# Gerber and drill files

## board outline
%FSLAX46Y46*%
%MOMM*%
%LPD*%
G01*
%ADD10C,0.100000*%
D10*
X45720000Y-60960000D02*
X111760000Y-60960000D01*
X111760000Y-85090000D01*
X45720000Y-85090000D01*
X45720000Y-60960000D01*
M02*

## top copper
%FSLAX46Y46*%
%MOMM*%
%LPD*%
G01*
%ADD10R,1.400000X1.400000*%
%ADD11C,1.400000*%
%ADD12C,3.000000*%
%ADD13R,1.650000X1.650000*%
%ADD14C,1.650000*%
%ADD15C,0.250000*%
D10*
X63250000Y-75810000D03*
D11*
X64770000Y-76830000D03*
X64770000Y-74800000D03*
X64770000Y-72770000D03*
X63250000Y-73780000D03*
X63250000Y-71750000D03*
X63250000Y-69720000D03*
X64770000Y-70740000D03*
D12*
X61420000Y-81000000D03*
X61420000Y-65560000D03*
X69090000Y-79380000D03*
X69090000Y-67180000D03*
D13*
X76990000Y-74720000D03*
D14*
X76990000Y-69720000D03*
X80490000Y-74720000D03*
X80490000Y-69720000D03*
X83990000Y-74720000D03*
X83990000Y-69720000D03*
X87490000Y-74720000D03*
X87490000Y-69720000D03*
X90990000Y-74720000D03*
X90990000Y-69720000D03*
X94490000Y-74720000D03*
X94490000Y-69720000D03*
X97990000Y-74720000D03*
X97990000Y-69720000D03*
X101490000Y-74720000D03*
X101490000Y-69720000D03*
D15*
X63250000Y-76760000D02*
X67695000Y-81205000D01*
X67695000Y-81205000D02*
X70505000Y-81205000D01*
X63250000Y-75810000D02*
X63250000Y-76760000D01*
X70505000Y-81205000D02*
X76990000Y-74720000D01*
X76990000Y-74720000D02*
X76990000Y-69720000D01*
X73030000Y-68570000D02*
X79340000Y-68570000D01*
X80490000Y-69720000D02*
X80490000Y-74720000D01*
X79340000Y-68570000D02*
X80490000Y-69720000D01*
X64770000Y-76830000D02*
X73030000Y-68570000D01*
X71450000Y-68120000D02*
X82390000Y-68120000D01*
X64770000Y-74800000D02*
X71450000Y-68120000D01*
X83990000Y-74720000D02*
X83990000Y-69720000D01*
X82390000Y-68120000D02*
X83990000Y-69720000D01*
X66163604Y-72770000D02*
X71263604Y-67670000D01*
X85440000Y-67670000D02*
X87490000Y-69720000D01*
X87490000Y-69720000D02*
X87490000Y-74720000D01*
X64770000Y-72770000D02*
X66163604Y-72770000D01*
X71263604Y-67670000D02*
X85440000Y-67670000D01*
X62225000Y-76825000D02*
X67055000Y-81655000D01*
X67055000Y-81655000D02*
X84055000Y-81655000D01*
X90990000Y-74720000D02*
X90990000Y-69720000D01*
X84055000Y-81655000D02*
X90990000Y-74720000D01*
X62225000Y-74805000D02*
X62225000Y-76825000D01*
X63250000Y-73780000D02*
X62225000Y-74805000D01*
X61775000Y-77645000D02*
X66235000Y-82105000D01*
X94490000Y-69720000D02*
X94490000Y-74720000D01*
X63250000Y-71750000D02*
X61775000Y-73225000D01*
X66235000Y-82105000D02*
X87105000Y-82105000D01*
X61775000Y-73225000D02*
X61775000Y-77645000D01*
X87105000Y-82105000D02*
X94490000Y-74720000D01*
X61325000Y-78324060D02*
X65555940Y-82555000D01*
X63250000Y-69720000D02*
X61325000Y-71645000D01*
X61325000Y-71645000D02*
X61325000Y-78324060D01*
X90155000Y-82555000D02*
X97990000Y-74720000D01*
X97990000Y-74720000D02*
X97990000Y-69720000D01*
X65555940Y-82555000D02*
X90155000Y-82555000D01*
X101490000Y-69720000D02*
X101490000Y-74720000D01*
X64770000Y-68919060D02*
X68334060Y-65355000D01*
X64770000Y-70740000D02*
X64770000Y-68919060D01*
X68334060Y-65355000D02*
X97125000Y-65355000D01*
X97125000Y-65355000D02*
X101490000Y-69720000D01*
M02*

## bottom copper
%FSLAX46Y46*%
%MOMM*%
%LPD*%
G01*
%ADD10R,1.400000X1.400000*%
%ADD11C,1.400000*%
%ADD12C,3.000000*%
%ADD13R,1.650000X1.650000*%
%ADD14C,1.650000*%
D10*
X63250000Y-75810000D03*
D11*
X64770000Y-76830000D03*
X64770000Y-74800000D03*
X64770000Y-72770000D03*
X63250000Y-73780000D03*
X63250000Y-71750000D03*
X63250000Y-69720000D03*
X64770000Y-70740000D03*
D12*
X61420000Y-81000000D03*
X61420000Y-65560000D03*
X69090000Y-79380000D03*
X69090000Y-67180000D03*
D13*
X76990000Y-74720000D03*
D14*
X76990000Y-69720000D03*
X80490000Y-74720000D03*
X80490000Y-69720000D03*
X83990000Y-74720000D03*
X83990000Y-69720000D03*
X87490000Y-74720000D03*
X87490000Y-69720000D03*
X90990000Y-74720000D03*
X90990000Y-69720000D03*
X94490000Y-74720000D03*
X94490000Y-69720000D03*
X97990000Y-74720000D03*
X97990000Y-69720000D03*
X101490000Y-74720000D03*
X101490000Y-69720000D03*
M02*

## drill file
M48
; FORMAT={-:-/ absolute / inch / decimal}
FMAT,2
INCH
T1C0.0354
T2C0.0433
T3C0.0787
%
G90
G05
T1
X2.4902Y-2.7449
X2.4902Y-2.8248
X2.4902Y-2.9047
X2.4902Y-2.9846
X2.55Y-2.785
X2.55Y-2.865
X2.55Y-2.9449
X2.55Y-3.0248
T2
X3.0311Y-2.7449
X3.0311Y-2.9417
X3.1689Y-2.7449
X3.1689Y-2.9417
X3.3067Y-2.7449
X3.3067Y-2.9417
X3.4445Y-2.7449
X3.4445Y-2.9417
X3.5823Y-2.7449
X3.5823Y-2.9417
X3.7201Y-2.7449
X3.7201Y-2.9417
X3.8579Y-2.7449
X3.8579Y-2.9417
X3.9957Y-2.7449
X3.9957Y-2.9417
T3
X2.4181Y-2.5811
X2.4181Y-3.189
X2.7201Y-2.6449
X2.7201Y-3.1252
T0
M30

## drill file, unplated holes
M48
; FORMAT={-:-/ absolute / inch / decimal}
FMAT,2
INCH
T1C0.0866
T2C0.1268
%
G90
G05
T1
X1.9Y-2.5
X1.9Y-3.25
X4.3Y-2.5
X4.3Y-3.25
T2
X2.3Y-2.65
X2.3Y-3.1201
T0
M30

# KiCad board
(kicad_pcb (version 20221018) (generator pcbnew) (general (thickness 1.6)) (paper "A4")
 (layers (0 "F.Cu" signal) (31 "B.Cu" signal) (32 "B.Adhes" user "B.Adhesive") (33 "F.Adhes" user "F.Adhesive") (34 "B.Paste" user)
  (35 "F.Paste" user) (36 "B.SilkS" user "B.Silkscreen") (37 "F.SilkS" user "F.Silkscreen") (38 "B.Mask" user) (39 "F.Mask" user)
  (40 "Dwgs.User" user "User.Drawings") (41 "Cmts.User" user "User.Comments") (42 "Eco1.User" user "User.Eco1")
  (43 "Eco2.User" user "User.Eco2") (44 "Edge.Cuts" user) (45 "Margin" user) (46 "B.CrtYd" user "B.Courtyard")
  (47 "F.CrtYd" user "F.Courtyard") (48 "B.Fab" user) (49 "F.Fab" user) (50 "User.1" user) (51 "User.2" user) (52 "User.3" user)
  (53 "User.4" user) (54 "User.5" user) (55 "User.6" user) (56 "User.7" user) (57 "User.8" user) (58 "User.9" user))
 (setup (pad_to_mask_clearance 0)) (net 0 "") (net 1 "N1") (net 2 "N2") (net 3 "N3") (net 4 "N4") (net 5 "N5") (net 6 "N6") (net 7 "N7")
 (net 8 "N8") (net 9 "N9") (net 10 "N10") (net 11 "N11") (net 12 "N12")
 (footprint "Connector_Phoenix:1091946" (layer "F.Cu") (at 63.25 75.81 -90)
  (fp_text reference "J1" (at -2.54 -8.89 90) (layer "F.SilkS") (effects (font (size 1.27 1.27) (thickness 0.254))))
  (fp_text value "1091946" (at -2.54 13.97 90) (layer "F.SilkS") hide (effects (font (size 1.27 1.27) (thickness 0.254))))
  (pad "" np_thru_hole circle (at -8.5 4.83 270) (size 3.22 3.22) (drill 3.22) (layers "*.Cu" "*.Mask"))
  (pad "" np_thru_hole circle (at 3.44 4.83 270) (size 3.22 3.22) (drill 3.22) (layers "*.Cu" "*.Mask"))
  (pad "1" thru_hole rect (at 0 0 270) (size 1.4 1.4) (drill 0.9) (layers "*.Cu" "*.Mask") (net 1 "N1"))
  (pad "2" thru_hole circle (at 1.02 -1.52 270) (size 1.4 1.4) (drill 0.9) (layers "*.Cu" "*.Mask") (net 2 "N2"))
  (pad "3" thru_hole circle (at -1.01 -1.52 270) (size 1.4 1.4) (drill 0.9) (layers "*.Cu" "*.Mask") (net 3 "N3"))
  (pad "4" thru_hole circle (at -3.04 -1.52 270) (size 1.4 1.4) (drill 0.9) (layers "*.Cu" "*.Mask") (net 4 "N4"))
  (pad "5" thru_hole circle (at -2.03 0 270) (size 1.4 1.4) (drill 0.9) (layers "*.Cu" "*.Mask") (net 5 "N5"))
  (pad "6" thru_hole circle (at -4.06 0 270) (size 1.4 1.4) (drill 0.9) (layers "*.Cu" "*.Mask") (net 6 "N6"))
  (pad "7" thru_hole circle (at -6.09 0 270) (size 1.4 1.4) (drill 0.9) (layers "*.Cu" "*.Mask") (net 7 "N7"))
  (pad "8" thru_hole circle (at -5.07 -1.52 270) (size 1.4 1.4) (drill 0.9) (layers "*.Cu" "*.Mask") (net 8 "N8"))
  (pad "MH1" thru_hole circle (at 5.19 1.83 270) (size 3 3) (drill 2) (layers "*.Cu" "*.Mask") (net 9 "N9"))
  (pad "MH2" thru_hole circle (at -10.25 1.83 270) (size 3 3) (drill 2) (layers "*.Cu" "*.Mask") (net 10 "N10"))
  (pad "MH3" thru_hole circle (at 3.57 -5.84 270) (size 3 3) (drill 2) (layers "*.Cu" "*.Mask") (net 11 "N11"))
  (pad "MH4" thru_hole circle (at -8.63 -5.84 270) (size 3 3) (drill 2) (layers "*.Cu" "*.Mask") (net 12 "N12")))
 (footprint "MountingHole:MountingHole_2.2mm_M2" (layer "F.Cu") (at 109.22 63.5)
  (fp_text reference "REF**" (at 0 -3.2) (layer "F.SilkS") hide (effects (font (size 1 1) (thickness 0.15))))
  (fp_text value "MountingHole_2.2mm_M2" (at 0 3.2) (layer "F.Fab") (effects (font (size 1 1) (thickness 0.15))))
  (pad "" np_thru_hole circle (at 0 0) (size 2.2 2.2) (drill 2.2) (layers "F&B.Cu" "*.Mask")))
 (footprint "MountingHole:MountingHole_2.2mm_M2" (layer "F.Cu") (at 109.22 82.55)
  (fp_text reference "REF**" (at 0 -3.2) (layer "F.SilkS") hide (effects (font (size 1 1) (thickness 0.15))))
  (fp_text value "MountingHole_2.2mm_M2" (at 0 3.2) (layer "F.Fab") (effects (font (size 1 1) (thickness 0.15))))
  (pad "" np_thru_hole circle (at 0 0) (size 2.2 2.2) (drill 2.2) (layers "F&B.Cu" "*.Mask")))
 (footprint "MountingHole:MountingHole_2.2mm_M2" (layer "F.Cu") (at 48.26 63.5)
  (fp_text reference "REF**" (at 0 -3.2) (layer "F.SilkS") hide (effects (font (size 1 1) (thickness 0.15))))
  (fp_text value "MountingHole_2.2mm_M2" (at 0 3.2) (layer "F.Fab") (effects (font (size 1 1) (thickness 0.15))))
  (pad "" np_thru_hole circle (at 0 0) (size 2.2 2.2) (drill 2.2) (layers "F&B.Cu" "*.Mask")))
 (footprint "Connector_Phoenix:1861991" (layer "F.Cu") (at 76.99 74.72)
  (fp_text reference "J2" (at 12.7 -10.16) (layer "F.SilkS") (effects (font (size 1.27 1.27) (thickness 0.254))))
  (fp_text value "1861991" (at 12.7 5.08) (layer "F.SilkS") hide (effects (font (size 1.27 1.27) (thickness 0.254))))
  (pad "1" thru_hole rect (at 0 0) (size 1.65 1.65) (drill 1.1) (layers "*.Cu" "*.Mask") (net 1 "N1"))
  (pad "2" thru_hole circle (at 0 -5) (size 1.65 1.65) (drill 1.1) (layers "*.Cu" "*.Mask") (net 1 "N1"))
  (pad "3" thru_hole circle (at 3.5 0) (size 1.65 1.65) (drill 1.1) (layers "*.Cu" "*.Mask") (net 2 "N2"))
  (pad "4" thru_hole circle (at 3.5 -5) (size 1.65 1.65) (drill 1.1) (layers "*.Cu" "*.Mask") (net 2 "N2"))
  (pad "5" thru_hole circle (at 7 0) (size 1.65 1.65) (drill 1.1) (layers "*.Cu" "*.Mask") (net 3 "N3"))
  (pad "6" thru_hole circle (at 7 -5) (size 1.65 1.65) (drill 1.1) (layers "*.Cu" "*.Mask") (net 3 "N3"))
  (pad "7" thru_hole circle (at 10.5 0) (size 1.65 1.65) (drill 1.1) (layers "*.Cu" "*.Mask") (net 4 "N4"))
  (pad "8" thru_hole circle (at 10.5 -5) (size 1.65 1.65) (drill 1.1) (layers "*.Cu" "*.Mask") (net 4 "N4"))
  (pad "9" thru_hole circle (at 14 0) (size 1.65 1.65) (drill 1.1) (layers "*.Cu" "*.Mask") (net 5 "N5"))
  (pad "10" thru_hole circle (at 14 -5) (size 1.65 1.65) (drill 1.1) (layers "*.Cu" "*.Mask") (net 5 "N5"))
  (pad "11" thru_hole circle (at 17.5 0) (size 1.65 1.65) (drill 1.1) (layers "*.Cu" "*.Mask") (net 6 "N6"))
  (pad "12" thru_hole circle (at 17.5 -5) (size 1.65 1.65) (drill 1.1) (layers "*.Cu" "*.Mask") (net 6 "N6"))
  (pad "13" thru_hole circle (at 21 0) (size 1.65 1.65) (drill 1.1) (layers "*.Cu" "*.Mask") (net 7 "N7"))
  (pad "14" thru_hole circle (at 21 -5) (size 1.65 1.65) (drill 1.1) (layers "*.Cu" "*.Mask") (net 7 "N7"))
  (pad "15" thru_hole circle (at 24.5 0) (size 1.65 1.65) (drill 1.1) (layers "*.Cu" "*.Mask") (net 8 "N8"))
  (pad "16" thru_hole circle (at 24.5 -5) (size 1.65 1.65) (drill 1.1) (layers "*.Cu" "*.Mask") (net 8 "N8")))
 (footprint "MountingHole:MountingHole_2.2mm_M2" (layer "F.Cu") (at 48.26 82.55)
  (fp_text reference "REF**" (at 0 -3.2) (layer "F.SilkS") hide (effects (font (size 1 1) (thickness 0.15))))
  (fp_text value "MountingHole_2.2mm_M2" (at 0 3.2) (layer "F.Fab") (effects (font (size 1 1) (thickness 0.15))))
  (pad "" np_thru_hole circle (at 0 0) (size 2.2 2.2) (drill 2.2) (layers "F&B.Cu" "*.Mask")))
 (gr_rect (start 45.72 60.96) (end 111.76 85.09) (stroke (width 0.1) (type default)) (fill none) (layer "Edge.Cuts"))
 (segment (start 63.25 76.76) (end 67.695 81.205) (width 0.25) (layer "F.Cu") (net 1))
 (segment (start 67.695 81.205) (end 70.505 81.205) (width 0.25) (layer "F.Cu") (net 1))
 (segment (start 63.25 75.81) (end 63.25 76.76) (width 0.25) (layer "F.Cu") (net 1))
 (segment (start 70.505 81.205) (end 76.99 74.72) (width 0.25) (layer "F.Cu") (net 1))
 (segment (start 76.99 74.72) (end 76.99 69.72) (width 0.25) (layer "F.Cu") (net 1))
 (segment (start 73.03 68.57) (end 79.34 68.57) (width 0.25) (layer "F.Cu") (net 2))
 (segment (start 80.49 69.72) (end 80.49 74.72) (width 0.25) (layer "F.Cu") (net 2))
 (segment (start 79.34 68.57) (end 80.49 69.72) (width 0.25) (layer "F.Cu") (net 2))
 (segment (start 64.77 76.83) (end 73.03 68.57) (width 0.25) (layer "F.Cu") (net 2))
 (segment (start 71.45 68.12) (end 82.39 68.12) (width 0.25) (layer "F.Cu") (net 3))
 (segment (start 64.77 74.8) (end 71.45 68.12) (width 0.25) (layer "F.Cu") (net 3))
 (segment (start 83.99 74.72) (end 83.99 69.72) (width 0.25) (layer "F.Cu") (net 3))
 (segment (start 82.39 68.12) (end 83.99 69.72) (width 0.25) (layer "F.Cu") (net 3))
 (segment (start 66.163604 72.77) (end 71.263604 67.67) (width 0.25) (layer "F.Cu") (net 4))
 (segment (start 85.44 67.67) (end 87.49 69.72) (width 0.25) (layer "F.Cu") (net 4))
 (segment (start 87.49 69.72) (end 87.49 74.72) (width 0.25) (layer "F.Cu") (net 4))
 (segment (start 64.77 72.77) (end 66.163604 72.77) (width 0.25) (layer "F.Cu") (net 4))
 (segment (start 71.263604 67.67) (end 85.44 67.67) (width 0.25) (layer "F.Cu") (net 4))
 (segment (start 62.225 76.825) (end 67.055 81.655) (width 0.25) (layer "F.Cu") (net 5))
 (segment (start 67.055 81.655) (end 84.055 81.655) (width 0.25) (layer "F.Cu") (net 5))
 (segment (start 90.99 74.72) (end 90.99 69.72) (width 0.25) (layer "F.Cu") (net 5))
 (segment (start 84.055 81.655) (end 90.99 74.72) (width 0.25) (layer "F.Cu") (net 5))
 (segment (start 62.225 74.805) (end 62.225 76.825) (width 0.25) (layer "F.Cu") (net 5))
 (segment (start 63.25 73.78) (end 62.225 74.805) (width 0.25) (layer "F.Cu") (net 5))
 (segment (start 61.775 77.645) (end 66.235 82.105) (width 0.25) (layer "F.Cu") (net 6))
 (segment (start 94.49 69.72) (end 94.49 74.72) (width 0.25) (layer "F.Cu") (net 6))
 (segment (start 63.25 71.75) (end 61.775 73.225) (width 0.25) (layer "F.Cu") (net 6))
 (segment (start 66.235 82.105) (end 87.105 82.105) (width 0.25) (layer "F.Cu") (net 6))
 (segment (start 61.775 73.225) (end 61.775 77.645) (width 0.25) (layer "F.Cu") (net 6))
 (segment (start 87.105 82.105) (end 94.49 74.72) (width 0.25) (layer "F.Cu") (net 6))
 (segment (start 61.325 78.32406) (end 65.55594 82.555) (width 0.25) (layer "F.Cu") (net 7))
 (segment (start 63.25 69.72) (end 61.325 71.645) (width 0.25) (layer "F.Cu") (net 7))
 (segment (start 61.325 71.645) (end 61.325 78.32406) (width 0.25) (layer "F.Cu") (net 7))
 (segment (start 90.155 82.555) (end 97.99 74.72) (width 0.25) (layer "F.Cu") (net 7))
 (segment (start 97.99 74.72) (end 97.99 69.72) (width 0.25) (layer "F.Cu") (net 7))
 (segment (start 65.55594 82.555) (end 90.155 82.555) (width 0.25) (layer "F.Cu") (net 7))
 (segment (start 101.49 69.72) (end 101.49 74.72) (width 0.25) (layer "F.Cu") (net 8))
 (segment (start 64.77 68.91906) (end 68.33406 65.355) (width 0.25) (layer "F.Cu") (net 8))
 (segment (start 64.77 70.74) (end 64.77 68.91906) (width 0.25) (layer "F.Cu") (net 8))
 (segment (start 68.33406 65.355) (end 97.125 65.355) (width 0.25) (layer "F.Cu") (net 8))
 (segment (start 97.125 65.355) (end 101.49 69.72) (width 0.25) (layer "F.Cu") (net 8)))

